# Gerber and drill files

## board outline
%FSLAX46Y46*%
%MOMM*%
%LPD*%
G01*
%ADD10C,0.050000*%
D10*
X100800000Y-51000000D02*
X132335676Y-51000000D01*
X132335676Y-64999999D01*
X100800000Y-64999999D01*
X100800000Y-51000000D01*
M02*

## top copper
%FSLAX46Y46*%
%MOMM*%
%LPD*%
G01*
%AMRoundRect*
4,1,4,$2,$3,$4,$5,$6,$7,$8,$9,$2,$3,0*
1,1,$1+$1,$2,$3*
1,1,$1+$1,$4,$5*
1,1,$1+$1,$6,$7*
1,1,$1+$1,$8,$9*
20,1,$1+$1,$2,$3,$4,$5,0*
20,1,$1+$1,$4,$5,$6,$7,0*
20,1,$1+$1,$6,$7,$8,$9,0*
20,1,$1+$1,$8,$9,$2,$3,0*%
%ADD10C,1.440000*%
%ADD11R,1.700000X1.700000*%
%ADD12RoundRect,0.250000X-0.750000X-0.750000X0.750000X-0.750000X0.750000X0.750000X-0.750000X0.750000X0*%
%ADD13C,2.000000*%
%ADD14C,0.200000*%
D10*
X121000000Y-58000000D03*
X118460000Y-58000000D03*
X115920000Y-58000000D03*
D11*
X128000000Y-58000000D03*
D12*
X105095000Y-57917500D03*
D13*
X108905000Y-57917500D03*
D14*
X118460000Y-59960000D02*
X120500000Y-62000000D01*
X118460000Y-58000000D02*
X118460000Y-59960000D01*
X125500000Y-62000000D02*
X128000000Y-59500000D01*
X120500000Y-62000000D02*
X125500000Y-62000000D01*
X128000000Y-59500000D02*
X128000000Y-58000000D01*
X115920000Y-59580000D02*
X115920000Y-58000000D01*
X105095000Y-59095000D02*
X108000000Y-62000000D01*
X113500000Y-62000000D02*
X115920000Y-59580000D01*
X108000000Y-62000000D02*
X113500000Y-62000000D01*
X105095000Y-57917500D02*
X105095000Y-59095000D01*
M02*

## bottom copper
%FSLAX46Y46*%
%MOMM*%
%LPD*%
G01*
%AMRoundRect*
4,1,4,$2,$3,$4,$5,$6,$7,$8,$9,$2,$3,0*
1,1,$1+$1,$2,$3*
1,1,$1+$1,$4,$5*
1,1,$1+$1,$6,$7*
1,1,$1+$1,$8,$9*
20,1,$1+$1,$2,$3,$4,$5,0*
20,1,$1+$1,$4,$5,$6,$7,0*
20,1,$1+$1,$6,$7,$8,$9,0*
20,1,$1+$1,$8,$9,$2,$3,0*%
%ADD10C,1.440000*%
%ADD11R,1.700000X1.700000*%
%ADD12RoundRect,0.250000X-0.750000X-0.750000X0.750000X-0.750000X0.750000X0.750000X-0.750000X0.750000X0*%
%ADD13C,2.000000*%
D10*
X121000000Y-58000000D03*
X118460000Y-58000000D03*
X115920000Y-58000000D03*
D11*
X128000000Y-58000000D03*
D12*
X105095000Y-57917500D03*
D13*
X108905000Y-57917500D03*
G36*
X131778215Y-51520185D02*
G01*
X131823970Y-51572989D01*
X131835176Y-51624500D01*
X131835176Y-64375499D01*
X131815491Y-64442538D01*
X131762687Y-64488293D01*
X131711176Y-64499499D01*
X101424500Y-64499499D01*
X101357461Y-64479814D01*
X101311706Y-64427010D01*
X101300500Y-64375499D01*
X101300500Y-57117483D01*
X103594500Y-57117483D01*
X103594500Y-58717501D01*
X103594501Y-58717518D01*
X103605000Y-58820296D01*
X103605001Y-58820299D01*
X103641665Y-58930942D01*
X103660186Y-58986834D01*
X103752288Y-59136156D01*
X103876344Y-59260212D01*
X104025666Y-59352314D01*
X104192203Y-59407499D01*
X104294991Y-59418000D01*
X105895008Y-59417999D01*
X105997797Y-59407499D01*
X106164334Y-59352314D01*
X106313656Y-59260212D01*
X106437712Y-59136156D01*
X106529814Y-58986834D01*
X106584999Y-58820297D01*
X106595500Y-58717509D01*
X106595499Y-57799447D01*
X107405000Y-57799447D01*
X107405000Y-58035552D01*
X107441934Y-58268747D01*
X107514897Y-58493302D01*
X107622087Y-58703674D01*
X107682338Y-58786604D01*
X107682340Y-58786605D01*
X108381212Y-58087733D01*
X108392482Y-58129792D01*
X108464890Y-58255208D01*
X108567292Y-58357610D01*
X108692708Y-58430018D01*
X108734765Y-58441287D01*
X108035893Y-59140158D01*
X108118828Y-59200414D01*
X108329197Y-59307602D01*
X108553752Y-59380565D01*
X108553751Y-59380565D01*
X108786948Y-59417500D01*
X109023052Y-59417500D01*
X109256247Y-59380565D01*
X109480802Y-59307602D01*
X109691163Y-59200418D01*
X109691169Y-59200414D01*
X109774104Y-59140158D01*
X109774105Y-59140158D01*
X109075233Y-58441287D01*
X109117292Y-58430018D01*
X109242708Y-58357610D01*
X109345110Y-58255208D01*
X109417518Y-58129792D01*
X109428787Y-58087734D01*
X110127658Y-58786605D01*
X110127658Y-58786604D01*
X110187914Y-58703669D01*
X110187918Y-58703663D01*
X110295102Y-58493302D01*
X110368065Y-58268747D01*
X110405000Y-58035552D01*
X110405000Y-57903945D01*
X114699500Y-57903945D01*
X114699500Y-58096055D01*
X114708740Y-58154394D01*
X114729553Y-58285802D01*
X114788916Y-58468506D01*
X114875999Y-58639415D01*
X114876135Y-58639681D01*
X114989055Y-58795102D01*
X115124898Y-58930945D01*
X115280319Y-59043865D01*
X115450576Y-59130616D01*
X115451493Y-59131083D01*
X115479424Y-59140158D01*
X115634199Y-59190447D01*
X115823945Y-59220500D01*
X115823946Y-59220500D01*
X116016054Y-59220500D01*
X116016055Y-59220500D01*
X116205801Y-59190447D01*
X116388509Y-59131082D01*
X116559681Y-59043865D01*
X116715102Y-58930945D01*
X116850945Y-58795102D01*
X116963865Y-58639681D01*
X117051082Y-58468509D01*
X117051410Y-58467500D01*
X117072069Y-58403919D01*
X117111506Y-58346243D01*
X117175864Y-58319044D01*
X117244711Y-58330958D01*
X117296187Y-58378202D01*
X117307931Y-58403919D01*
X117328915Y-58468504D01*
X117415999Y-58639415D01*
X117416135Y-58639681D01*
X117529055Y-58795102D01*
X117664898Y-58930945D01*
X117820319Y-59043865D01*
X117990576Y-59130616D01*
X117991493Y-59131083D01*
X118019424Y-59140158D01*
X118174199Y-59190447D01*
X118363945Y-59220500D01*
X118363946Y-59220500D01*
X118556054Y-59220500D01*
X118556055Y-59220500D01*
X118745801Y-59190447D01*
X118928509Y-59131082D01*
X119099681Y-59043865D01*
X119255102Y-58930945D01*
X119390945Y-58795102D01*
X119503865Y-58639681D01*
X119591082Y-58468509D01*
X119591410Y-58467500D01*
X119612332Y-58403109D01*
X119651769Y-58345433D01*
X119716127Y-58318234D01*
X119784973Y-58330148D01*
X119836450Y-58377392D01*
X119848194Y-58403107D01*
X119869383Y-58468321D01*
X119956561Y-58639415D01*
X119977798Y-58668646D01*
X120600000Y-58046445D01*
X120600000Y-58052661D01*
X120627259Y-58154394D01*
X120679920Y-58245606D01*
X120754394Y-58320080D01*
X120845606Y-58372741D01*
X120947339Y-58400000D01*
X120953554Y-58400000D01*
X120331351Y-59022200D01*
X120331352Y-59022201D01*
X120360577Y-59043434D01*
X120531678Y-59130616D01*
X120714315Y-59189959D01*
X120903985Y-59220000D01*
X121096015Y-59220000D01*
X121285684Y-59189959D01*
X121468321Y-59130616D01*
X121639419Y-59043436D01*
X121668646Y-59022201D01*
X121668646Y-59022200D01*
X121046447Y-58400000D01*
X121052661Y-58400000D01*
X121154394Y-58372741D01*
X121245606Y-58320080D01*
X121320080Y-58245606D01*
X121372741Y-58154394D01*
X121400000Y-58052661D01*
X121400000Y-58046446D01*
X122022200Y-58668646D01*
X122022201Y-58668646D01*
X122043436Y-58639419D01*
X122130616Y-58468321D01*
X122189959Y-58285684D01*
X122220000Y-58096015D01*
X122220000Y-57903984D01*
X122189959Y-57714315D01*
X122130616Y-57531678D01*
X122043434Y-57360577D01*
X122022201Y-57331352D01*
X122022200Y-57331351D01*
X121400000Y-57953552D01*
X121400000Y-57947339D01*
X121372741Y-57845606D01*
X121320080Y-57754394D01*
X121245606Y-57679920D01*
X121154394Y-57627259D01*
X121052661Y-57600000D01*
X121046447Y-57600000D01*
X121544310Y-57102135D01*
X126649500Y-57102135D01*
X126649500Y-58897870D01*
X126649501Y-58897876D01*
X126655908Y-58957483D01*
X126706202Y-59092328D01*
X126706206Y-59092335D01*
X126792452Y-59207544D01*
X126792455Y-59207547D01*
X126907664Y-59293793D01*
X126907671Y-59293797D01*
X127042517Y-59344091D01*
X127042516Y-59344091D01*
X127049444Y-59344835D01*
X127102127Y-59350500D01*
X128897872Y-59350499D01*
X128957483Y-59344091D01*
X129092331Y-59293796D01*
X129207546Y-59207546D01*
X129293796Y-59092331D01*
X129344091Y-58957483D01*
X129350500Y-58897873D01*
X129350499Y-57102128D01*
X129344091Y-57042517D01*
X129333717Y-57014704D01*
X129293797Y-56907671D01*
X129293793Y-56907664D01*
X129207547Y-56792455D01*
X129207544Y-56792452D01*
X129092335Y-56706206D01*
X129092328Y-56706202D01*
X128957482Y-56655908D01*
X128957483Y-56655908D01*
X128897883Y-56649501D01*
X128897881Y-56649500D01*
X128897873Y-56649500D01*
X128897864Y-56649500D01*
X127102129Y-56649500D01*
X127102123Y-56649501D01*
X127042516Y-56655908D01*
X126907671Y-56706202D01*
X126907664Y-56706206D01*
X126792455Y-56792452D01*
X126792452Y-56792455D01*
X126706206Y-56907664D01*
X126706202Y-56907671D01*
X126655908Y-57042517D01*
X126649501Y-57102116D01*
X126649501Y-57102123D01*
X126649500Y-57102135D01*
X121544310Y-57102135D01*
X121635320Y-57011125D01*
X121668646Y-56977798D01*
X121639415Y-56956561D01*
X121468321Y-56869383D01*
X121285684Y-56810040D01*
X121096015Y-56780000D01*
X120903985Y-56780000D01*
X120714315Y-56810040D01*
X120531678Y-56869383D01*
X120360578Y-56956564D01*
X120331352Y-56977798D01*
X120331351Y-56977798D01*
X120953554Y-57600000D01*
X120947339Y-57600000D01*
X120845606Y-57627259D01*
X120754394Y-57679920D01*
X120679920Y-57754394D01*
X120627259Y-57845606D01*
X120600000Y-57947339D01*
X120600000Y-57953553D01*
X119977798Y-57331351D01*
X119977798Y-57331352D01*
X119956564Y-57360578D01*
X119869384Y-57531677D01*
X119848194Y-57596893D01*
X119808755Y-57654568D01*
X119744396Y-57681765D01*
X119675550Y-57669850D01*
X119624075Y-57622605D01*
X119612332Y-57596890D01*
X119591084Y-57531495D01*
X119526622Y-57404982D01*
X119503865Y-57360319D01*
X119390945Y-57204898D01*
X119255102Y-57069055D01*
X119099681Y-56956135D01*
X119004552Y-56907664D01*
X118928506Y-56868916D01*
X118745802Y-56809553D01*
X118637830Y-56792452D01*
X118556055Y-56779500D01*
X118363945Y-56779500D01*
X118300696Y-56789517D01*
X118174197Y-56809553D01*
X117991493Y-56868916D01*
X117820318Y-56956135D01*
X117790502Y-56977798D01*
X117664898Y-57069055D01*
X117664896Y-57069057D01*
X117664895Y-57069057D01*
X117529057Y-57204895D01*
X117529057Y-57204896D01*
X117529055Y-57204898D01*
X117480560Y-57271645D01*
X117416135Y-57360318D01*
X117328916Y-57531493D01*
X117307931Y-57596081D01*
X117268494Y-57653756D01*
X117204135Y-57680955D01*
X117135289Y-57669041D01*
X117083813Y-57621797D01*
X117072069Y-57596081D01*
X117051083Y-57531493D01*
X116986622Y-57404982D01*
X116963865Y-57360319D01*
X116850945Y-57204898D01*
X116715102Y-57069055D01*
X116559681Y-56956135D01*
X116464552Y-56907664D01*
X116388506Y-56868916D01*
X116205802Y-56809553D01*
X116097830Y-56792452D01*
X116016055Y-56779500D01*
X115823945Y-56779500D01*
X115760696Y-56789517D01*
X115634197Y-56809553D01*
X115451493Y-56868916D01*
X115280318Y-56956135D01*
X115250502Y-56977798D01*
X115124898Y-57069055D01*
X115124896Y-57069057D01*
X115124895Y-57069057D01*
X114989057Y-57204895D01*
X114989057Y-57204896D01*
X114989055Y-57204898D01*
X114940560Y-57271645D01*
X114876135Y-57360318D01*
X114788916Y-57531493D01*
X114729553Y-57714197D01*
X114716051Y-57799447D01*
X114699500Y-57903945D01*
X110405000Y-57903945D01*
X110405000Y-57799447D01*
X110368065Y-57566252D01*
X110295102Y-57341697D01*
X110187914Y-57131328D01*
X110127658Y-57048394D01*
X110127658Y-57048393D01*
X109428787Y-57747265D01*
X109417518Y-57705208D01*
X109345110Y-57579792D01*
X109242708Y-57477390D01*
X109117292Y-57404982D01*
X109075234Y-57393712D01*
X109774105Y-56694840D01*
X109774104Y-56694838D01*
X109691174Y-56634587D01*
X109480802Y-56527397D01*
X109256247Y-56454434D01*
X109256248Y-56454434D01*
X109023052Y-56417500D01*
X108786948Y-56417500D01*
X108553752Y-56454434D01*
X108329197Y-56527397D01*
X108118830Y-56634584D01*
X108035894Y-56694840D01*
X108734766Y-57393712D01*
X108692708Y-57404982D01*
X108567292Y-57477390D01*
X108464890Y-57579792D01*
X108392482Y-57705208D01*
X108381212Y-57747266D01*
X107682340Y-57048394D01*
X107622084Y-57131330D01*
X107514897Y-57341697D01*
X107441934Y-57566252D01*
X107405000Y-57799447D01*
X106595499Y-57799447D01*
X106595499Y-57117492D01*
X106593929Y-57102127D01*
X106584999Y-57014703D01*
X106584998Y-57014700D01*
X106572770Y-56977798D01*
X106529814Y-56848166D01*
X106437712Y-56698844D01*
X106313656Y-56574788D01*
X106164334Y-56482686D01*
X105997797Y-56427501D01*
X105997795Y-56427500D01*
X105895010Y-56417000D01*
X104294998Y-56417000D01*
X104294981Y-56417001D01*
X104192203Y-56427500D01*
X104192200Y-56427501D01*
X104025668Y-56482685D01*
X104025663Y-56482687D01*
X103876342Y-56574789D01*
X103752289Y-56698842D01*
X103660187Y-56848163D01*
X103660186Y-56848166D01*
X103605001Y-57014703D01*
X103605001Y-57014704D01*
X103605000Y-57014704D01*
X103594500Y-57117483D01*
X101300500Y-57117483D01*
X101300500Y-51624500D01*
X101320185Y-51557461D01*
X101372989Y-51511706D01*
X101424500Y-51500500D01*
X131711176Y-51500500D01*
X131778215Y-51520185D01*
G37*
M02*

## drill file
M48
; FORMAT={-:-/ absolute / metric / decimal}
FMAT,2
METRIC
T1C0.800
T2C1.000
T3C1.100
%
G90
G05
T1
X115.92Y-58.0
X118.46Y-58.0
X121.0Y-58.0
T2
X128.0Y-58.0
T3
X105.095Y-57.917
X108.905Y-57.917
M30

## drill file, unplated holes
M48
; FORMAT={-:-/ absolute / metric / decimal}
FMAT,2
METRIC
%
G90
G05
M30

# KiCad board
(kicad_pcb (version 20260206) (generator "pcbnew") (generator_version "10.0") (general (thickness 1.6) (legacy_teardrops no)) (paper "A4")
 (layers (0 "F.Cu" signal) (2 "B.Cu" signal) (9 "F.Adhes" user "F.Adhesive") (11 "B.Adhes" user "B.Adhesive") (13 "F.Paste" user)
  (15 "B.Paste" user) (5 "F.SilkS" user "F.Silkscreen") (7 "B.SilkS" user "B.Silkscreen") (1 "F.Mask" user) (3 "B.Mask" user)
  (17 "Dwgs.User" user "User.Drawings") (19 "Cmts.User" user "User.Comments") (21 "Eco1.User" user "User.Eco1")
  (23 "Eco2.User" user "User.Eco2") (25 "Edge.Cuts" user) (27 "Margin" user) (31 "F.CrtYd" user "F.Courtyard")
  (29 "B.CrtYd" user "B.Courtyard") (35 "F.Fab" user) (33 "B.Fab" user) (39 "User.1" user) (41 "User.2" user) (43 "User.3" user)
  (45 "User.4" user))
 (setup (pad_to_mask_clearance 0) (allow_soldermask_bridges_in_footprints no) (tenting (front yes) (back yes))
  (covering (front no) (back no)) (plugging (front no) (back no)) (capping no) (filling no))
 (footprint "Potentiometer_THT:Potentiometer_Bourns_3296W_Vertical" (layer "F.Cu") (at 121 58)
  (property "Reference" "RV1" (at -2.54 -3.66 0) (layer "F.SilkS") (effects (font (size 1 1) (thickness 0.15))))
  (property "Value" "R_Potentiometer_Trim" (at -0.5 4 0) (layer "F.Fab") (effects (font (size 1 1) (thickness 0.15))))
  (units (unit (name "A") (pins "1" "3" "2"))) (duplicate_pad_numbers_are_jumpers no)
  (pad "1" thru_hole circle (at 0 0) (size 1.44 1.44) (drill 0.8) (layers "*.Cu" "*.Mask") (remove_unused_layers no) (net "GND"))
  (pad "2" thru_hole circle (at -2.54 0) (size 1.44 1.44) (drill 0.8) (layers "*.Cu" "*.Mask") (remove_unused_layers no)
   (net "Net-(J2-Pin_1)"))
  (pad "3" thru_hole circle (at -5.08 0) (size 1.44 1.44) (drill 0.8) (layers "*.Cu" "*.Mask") (remove_unused_layers no) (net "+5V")))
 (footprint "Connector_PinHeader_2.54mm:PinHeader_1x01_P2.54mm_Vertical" (layer "F.Cu") (at 128 58)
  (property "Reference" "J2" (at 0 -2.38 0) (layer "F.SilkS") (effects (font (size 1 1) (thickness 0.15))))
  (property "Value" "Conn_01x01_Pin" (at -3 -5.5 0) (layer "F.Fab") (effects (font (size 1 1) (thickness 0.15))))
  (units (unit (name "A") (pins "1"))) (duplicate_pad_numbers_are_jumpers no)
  (pad "1" thru_hole rect (at 0 0) (size 1.7 1.7) (drill 1) (layers "*.Cu" "*.Mask") (remove_unused_layers no) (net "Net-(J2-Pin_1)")))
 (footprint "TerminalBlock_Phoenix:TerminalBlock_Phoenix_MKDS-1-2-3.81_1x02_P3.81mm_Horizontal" (layer "F.Cu") (at 105.095 57.9175)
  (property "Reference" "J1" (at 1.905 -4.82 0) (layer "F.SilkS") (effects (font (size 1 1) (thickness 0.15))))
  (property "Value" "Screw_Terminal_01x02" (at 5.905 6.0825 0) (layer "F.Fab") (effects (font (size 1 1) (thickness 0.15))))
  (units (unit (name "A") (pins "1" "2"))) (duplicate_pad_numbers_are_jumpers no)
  (pad "1" thru_hole roundrect (at 0 0) (size 2 2) (drill 1.1) (layers "*.Cu" "*.Mask") (remove_unused_layers no) (roundrect_rratio 0.125)
   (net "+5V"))
  (pad "2" thru_hole circle (at 3.81 0) (size 2 2) (drill 1.1) (layers "*.Cu" "*.Mask") (remove_unused_layers no) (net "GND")))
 (gr_rect (start 100.8 51) (end 132.335676 64.999999) (stroke (width 0.05) (type default)) (fill no) (layer "Edge.Cuts"))
 (segment (start 118.46 59.96) (end 120.5 62) (width 0.2) (layer "F.Cu") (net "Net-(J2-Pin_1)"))
 (segment (start 118.46 58) (end 118.46 59.96) (width 0.2) (layer "F.Cu") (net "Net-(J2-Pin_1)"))
 (segment (start 125.5 62) (end 128 59.5) (width 0.2) (layer "F.Cu") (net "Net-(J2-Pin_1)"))
 (segment (start 120.5 62) (end 125.5 62) (width 0.2) (layer "F.Cu") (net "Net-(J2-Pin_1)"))
 (segment (start 128 59.5) (end 128 58) (width 0.2) (layer "F.Cu") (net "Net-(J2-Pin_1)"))
 (segment (start 115.92 59.58) (end 115.92 58) (width 0.2) (layer "F.Cu") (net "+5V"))
 (segment (start 105.095 59.095) (end 108 62) (width 0.2) (layer "F.Cu") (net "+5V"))
 (segment (start 113.5 62) (end 115.92 59.58) (width 0.2) (layer "F.Cu") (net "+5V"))
 (segment (start 108 62) (end 113.5 62) (width 0.2) (layer "F.Cu") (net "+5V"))
 (segment (start 105.095 57.9175) (end 105.095 59.095) (width 0.2) (layer "F.Cu") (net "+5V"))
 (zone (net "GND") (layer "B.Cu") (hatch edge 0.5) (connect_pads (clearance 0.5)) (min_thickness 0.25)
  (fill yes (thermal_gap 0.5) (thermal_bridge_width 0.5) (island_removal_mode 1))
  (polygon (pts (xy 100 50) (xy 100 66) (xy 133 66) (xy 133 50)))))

